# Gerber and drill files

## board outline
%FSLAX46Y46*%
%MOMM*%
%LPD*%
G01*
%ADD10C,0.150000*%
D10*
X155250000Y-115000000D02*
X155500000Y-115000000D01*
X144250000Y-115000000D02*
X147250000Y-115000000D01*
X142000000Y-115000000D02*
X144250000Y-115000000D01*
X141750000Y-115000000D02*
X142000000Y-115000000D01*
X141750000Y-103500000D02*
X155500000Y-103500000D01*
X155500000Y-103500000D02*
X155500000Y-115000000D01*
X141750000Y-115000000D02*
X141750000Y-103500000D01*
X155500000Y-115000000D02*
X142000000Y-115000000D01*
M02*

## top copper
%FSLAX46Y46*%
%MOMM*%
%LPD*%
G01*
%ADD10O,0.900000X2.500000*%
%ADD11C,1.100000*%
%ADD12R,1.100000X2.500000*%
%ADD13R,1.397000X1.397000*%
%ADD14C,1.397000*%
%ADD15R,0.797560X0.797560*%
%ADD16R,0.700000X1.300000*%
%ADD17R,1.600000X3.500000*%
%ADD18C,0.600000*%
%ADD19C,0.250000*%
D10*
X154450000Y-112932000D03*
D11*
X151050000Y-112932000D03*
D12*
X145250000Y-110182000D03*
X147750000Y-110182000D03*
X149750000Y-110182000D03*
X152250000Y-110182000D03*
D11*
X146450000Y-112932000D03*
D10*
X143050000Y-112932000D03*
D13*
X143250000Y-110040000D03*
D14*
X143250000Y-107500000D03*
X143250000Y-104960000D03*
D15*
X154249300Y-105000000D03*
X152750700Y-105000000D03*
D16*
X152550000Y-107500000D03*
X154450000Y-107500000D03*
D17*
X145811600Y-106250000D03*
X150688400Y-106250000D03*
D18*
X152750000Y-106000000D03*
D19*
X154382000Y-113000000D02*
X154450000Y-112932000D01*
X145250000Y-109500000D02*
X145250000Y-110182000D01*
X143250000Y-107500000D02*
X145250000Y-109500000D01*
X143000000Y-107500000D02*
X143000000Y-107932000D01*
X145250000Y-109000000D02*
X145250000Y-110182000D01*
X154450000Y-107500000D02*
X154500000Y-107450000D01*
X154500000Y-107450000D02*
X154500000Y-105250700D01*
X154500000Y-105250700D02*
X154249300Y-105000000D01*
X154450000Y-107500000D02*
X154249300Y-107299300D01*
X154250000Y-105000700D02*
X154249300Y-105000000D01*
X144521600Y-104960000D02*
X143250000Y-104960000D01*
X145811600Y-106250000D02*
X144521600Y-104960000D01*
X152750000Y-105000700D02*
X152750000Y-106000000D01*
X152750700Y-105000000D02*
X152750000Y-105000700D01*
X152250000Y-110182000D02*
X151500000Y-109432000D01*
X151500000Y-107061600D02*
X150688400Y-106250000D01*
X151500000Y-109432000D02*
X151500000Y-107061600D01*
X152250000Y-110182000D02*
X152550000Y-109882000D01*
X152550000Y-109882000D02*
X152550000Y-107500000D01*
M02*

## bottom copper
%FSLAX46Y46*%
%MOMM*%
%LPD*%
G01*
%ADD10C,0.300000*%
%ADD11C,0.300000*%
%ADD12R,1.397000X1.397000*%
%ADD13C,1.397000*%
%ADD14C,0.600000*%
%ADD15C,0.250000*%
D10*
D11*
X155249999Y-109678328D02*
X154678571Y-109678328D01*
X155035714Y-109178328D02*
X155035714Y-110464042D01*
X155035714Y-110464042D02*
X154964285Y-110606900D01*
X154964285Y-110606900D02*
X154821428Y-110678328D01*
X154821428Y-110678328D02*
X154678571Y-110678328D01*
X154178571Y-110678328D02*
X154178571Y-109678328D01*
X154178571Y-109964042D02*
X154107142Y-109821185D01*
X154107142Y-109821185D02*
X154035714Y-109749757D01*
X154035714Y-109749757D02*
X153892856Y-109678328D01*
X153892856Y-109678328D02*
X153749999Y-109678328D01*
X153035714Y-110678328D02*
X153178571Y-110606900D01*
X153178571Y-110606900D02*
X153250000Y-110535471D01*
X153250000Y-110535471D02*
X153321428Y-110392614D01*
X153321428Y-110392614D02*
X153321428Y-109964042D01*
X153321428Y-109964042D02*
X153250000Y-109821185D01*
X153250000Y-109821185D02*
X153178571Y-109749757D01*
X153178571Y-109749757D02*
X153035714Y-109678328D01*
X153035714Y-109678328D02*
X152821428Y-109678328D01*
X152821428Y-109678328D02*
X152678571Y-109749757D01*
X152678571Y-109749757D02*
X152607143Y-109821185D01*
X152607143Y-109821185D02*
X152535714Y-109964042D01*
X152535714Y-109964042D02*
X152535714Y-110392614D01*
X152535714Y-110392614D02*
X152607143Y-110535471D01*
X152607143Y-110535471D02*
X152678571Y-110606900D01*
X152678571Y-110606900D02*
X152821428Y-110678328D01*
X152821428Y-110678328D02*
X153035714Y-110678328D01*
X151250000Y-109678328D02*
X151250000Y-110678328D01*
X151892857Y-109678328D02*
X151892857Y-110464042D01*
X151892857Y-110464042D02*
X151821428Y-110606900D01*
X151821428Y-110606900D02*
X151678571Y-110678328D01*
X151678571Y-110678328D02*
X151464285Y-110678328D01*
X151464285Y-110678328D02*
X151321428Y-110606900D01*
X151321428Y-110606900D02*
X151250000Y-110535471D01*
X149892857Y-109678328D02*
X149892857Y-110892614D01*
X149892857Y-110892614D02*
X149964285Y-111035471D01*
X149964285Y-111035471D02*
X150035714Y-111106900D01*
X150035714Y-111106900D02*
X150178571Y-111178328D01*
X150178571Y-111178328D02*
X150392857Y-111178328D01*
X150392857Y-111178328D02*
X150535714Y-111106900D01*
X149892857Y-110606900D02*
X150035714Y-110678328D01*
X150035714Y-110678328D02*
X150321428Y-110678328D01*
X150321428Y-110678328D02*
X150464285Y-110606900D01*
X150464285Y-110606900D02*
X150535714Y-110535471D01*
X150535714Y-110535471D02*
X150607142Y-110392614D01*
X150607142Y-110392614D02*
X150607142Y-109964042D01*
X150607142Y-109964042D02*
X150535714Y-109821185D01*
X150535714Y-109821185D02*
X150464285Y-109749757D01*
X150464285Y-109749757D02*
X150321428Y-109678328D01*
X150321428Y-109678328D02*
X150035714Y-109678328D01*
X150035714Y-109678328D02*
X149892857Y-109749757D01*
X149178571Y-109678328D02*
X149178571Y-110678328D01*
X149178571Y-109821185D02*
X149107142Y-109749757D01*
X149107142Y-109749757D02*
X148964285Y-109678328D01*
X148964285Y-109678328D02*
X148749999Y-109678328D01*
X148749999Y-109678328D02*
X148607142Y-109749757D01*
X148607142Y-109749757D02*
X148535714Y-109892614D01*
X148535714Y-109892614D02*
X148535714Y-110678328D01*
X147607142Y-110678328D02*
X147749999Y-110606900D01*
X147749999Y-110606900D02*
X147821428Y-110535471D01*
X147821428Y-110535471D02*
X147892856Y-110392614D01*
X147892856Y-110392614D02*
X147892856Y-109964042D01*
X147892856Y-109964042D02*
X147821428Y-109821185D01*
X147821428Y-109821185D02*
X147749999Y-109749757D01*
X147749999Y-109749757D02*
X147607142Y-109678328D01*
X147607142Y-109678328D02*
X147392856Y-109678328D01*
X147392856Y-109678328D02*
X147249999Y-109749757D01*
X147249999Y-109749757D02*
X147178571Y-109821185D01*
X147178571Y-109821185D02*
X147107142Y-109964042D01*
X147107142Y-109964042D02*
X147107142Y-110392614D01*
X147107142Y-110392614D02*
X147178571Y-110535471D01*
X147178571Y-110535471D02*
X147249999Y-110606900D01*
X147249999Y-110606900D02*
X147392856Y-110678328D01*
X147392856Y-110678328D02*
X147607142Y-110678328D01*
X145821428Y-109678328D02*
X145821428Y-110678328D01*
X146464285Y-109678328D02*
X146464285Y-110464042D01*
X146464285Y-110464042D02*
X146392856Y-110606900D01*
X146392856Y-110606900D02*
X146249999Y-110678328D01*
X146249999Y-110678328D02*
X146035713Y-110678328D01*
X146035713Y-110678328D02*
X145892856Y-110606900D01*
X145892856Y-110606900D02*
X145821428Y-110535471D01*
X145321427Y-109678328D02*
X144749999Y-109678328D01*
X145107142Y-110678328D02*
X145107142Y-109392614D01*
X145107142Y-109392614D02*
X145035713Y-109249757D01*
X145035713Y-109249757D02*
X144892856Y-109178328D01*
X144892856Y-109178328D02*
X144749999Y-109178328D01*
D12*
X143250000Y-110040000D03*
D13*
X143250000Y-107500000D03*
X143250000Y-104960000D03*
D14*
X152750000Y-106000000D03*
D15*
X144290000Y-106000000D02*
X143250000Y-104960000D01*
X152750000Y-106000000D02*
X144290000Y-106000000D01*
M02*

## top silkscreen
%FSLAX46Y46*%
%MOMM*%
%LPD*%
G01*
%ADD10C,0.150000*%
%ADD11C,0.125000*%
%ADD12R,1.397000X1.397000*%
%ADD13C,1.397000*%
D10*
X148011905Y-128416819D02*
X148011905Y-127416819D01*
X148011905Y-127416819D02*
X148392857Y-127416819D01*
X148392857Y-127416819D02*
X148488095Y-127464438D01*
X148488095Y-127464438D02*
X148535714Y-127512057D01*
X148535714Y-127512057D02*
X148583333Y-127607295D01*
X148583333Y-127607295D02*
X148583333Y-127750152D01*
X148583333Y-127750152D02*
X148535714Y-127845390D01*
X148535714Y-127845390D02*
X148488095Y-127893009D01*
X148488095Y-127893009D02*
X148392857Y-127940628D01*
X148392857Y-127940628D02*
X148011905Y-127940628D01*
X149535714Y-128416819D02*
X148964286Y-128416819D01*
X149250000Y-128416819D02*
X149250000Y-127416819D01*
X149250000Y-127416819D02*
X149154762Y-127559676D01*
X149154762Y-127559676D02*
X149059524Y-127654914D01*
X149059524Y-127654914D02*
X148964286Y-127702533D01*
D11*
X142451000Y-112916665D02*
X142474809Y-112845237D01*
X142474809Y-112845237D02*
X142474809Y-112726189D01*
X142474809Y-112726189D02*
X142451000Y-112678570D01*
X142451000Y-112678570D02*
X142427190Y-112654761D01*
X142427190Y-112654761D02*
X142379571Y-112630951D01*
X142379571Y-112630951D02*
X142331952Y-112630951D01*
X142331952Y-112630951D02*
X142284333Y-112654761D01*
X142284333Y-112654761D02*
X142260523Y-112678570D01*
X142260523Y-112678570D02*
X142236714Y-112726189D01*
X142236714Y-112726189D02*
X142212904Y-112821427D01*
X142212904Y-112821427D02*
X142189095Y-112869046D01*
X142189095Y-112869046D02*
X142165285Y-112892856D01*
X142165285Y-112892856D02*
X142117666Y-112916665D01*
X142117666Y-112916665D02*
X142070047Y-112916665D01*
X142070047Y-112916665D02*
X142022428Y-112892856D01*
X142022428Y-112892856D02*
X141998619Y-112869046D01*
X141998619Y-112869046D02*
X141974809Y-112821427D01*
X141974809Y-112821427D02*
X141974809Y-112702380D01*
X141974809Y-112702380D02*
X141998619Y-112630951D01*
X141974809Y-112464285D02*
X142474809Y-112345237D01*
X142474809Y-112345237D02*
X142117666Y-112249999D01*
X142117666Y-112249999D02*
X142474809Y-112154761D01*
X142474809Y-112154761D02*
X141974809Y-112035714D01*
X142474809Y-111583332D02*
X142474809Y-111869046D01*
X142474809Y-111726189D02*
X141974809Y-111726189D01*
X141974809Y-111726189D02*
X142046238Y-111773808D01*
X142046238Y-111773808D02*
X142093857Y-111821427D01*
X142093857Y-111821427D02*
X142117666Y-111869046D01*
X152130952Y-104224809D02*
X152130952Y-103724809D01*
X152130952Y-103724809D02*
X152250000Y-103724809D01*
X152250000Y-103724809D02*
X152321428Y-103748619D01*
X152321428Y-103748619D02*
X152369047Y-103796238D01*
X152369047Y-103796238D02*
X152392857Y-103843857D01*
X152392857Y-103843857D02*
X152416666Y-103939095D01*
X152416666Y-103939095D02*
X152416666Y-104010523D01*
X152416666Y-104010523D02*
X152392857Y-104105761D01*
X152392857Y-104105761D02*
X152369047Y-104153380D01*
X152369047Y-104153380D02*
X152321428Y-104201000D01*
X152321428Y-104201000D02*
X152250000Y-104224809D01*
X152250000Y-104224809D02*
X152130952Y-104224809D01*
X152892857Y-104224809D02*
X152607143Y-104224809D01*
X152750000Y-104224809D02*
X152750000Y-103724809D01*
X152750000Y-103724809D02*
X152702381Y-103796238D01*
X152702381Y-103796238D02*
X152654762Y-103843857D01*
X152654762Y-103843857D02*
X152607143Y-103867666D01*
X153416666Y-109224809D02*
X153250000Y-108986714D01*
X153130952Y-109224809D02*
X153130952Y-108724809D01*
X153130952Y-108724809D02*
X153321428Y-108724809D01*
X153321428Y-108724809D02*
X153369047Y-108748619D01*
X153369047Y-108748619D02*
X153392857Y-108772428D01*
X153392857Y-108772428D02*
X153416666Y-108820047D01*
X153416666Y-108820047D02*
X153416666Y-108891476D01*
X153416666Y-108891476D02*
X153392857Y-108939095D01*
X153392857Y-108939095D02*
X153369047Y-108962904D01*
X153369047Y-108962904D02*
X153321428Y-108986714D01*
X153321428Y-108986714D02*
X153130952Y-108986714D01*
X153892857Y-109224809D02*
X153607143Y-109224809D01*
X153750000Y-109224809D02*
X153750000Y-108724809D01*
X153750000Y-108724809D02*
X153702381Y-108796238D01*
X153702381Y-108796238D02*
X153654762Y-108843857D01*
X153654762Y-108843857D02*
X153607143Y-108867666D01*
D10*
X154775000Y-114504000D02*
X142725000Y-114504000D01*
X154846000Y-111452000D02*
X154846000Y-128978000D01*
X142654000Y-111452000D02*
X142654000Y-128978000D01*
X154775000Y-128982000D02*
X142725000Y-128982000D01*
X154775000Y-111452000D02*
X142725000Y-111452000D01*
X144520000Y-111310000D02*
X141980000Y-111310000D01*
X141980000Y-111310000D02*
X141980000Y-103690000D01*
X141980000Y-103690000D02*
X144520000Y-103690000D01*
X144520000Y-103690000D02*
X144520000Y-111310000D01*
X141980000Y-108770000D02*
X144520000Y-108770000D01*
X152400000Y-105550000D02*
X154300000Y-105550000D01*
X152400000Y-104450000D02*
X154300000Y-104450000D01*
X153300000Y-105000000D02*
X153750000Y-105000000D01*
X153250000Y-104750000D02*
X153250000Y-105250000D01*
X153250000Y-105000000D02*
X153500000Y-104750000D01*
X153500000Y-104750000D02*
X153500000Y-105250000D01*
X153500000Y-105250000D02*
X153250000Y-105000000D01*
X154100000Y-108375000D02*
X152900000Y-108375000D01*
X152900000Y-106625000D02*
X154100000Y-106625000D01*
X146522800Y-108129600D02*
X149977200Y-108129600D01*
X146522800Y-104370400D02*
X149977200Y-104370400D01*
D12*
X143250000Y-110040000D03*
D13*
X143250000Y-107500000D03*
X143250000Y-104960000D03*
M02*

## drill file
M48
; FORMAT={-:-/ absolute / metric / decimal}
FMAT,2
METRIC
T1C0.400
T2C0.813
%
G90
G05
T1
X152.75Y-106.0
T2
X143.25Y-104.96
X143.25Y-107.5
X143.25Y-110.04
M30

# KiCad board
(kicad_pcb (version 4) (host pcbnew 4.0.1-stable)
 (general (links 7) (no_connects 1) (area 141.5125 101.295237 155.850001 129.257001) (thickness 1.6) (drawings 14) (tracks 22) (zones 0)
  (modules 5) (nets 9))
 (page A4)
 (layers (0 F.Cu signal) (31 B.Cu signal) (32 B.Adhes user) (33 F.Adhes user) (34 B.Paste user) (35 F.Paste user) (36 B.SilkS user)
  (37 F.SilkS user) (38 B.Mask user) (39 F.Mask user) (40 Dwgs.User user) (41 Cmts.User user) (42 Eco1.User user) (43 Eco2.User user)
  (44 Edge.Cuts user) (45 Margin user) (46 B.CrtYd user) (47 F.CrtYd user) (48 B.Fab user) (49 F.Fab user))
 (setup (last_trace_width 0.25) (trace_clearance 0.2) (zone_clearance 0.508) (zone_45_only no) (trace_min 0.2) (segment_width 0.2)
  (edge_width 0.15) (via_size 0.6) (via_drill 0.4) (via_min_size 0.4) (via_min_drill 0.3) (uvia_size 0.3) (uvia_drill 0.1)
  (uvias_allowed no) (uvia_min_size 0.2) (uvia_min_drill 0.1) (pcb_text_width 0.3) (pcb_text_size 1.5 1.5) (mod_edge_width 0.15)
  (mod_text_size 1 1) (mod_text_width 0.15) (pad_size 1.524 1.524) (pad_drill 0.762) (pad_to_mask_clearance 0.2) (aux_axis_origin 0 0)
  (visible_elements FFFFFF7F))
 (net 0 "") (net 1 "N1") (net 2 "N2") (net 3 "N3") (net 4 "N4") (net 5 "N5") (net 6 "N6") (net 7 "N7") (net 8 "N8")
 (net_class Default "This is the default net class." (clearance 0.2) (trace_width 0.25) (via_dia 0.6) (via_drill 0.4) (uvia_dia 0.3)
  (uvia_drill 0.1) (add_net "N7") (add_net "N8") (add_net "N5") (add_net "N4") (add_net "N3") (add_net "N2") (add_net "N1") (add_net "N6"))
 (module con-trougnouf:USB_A (layer F.Cu) (at 148.75 114.5)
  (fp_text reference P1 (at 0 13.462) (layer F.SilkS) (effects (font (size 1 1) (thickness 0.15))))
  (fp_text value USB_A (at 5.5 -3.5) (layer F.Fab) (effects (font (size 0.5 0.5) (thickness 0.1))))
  (fp_line (start 6.025 0.004) (end -6.025 0.004) (layer F.SilkS) (width 0.15))
  (fp_line (start 6.096 -3.048) (end 6.096 14.478) (layer F.SilkS) (width 0.15))
  (fp_line (start -6.096 -3.048) (end -6.096 14.478) (layer F.SilkS) (width 0.15))
  (fp_line (start 6.025 14.482) (end -6.025 14.482) (layer F.SilkS) (width 0.15))
  (fp_line (start 6.025 -3.048) (end -6.025 -3.048) (layer F.SilkS) (width 0.15))
  (pad 5 smd oval (at 5.7 -1.568) (size 0.9 2.5) (layers F.Cu F.Paste F.Mask) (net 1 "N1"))
  (pad "" smd circle (at 2.3 -1.568) (size 1.1 1.1) (layers F.Cu F.Paste F.Mask))
  (pad 4 smd rect (at -3.5 -4.318) (size 1.1 2.5) (layers F.Cu F.Paste F.Mask) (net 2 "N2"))
  (pad 3 smd rect (at -1 -4.318) (size 1.1 2.5) (layers F.Cu F.Paste F.Mask) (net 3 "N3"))
  (pad 2 smd rect (at 1 -4.318) (size 1.1 2.5) (layers F.Cu F.Paste F.Mask) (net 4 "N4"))
  (pad 1 smd rect (at 3.5 -4.318) (size 1.1 2.5) (layers F.Cu F.Paste F.Mask) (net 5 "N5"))
  (pad "" smd circle (at -2.3 -1.568) (size 1.1 1.1) (layers F.Cu F.Paste F.Mask))
  (pad 5 smd oval (at -5.7 -1.568) (size 0.9 2.5) (layers F.Cu F.Paste F.Mask) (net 1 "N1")))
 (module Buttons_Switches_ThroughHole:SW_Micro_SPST (layer F.Cu) (at 143.25 107.5 90)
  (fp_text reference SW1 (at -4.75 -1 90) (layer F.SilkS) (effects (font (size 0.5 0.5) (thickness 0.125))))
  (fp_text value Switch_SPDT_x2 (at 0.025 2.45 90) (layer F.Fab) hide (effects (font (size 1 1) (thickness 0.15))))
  (fp_line (start -3.81 1.27) (end -3.81 -1.27) (layer F.SilkS) (width 0.15))
  (fp_line (start -3.81 -1.27) (end 3.81 -1.27) (layer F.SilkS) (width 0.15))
  (fp_line (start 3.81 -1.27) (end 3.81 1.27) (layer F.SilkS) (width 0.15))
  (fp_line (start 3.81 1.27) (end -3.81 1.27) (layer F.SilkS) (width 0.15))
  (fp_line (start -1.27 -1.27) (end -1.27 1.27) (layer F.SilkS) (width 0.15))
  (pad 1 thru_hole rect (at -2.54 0 90) (size 1.397 1.397) (drill 0.8128) (layers *.Cu *.Mask F.SilkS) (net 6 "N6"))
  (pad 2 thru_hole circle (at 0 0 90) (size 1.397 1.397) (drill 0.8128) (layers *.Cu *.Mask F.SilkS) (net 2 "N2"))
  (pad 3 thru_hole circle (at 2.54 0 90) (size 1.397 1.397) (drill 0.8128) (layers *.Cu *.Mask F.SilkS) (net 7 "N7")))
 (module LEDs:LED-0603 (layer F.Cu) (at 153.5 105)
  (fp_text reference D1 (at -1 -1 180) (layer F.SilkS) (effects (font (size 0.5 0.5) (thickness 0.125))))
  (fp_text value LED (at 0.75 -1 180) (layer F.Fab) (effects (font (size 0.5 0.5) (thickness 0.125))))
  (fp_line (start -1.1 0.55) (end 0.8 0.55) (layer F.SilkS) (width 0.15))
  (fp_line (start -1.1 -0.55) (end 0.8 -0.55) (layer F.SilkS) (width 0.15))
  (fp_line (start -0.2 0) (end 0.25 0) (layer F.SilkS) (width 0.15))
  (fp_line (start -0.25 -0.25) (end -0.25 0.25) (layer F.SilkS) (width 0.15))
  (fp_line (start -0.25 0) (end 0 -0.25) (layer F.SilkS) (width 0.15))
  (fp_line (start 0 -0.25) (end 0 0.25) (layer F.SilkS) (width 0.15))
  (fp_line (start 0 0.25) (end -0.25 0) (layer F.SilkS) (width 0.15))
  (pad 2 smd rect (at 0.7493 0 180) (size 0.79756 0.79756) (layers F.Cu F.Paste F.Mask) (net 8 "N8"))
  (pad 1 smd rect (at -0.7493 0 180) (size 0.79756 0.79756) (layers F.Cu F.Paste F.Mask) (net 7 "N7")))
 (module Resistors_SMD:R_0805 (layer F.Cu) (at 153.5 107.5)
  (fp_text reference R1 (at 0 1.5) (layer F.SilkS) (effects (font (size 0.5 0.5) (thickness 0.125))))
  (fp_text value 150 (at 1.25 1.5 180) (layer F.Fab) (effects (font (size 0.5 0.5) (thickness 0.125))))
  (fp_line (start 0.6 0.875) (end -0.6 0.875) (layer F.SilkS) (width 0.15))
  (fp_line (start -0.6 -0.875) (end 0.6 -0.875) (layer F.SilkS) (width 0.15))
  (pad 1 smd rect (at -0.95 0) (size 0.7 1.3) (layers F.Cu F.Paste F.Mask) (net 5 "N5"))
  (pad 2 smd rect (at 0.95 0) (size 0.7 1.3) (layers F.Cu F.Paste F.Mask) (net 8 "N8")))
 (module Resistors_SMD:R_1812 (layer F.Cu) (at 148.25 106.25)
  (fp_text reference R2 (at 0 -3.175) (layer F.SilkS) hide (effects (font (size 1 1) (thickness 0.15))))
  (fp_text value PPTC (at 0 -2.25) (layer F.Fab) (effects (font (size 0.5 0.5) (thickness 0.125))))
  (fp_line (start -1.7272 1.8796) (end 1.7272 1.8796) (layer F.SilkS) (width 0.15))
  (fp_line (start -1.7272 -1.8796) (end 1.7272 -1.8796) (layer F.SilkS) (width 0.15))
  (pad 1 smd rect (at -2.4384 0) (size 1.6 3.5) (layers F.Cu F.Paste F.Mask) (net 7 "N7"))
  (pad 2 smd rect (at 2.4384 0) (size 1.6 3.5) (layers F.Cu F.Paste F.Mask) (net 5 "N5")))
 (gr_line (start 155.25 115) (end 155.5 115) (angle 90) (layer Edge.Cuts) (width 0.15))
 (gr_line (start 144.25 115) (end 147.25 115) (angle 90) (layer Edge.Cuts) (width 0.15))
 (gr_line (start 142 115) (end 144.25 115) (angle 90) (layer Edge.Cuts) (width 0.15))
 (gr_line (start 141.75 115) (end 142 115) (angle 90) (layer Edge.Cuts) (width 0.15))
 (gr_line (start 141.75 103.5) (end 155.5 103.5) (angle 90) (layer Edge.Cuts) (width 0.15))
 (gr_line (start 155.5 103.5) (end 155.5 115) (angle 90) (layer Edge.Cuts) (width 0.15))
 (gr_line (start 141.75 115) (end 141.75 103.5) (angle 90) (layer Edge.Cuts) (width 0.15))
 (gr_line (start 155.5 115) (end 142 115) (angle 90) (layer Edge.Cuts) (width 0.15))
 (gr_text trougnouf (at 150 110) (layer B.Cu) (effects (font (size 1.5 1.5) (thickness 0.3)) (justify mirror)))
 (segment (start 154.382 113) (end 154.45 112.932) (width 0.25) (layer F.Cu) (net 1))
 (segment (start 145.25 109.5) (end 145.25 110.182) (width 0.25) (layer F.Cu) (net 2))
 (segment (start 143.25 107.5) (end 145.25 109.5) (width 0.25) (layer F.Cu) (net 2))
 (segment (start 143 107.5) (end 143 107.932) (width 0.25) (layer F.Cu) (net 2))
 (segment (start 145.25 109) (end 145.25 110.182) (width 0.25) (layer F.Cu) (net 2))
 (segment (start 154.45 107.5) (end 154.5 107.45) (width 0.25) (layer F.Cu) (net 8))
 (segment (start 154.5 107.45) (end 154.5 105.2507) (width 0.25) (layer F.Cu) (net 8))
 (segment (start 154.5 105.2507) (end 154.2493 105) (width 0.25) (layer F.Cu) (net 8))
 (segment (start 154.45 107.5) (end 154.2493 107.2993) (width 0.25) (layer F.Cu) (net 8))
 (segment (start 154.25 105.0007) (end 154.2493 105) (width 0.25) (layer F.Cu) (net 8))
 (segment (start 144.5216 104.96) (end 143.25 104.96) (width 0.25) (layer F.Cu) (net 7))
 (segment (start 145.8116 106.25) (end 144.5216 104.96) (width 0.25) (layer F.Cu) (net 7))
 (segment (start 144.29 106) (end 143.25 104.96) (width 0.25) (layer B.Cu) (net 7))
 (segment (start 152.75 106) (end 144.29 106) (width 0.25) (layer B.Cu) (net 7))
 (via (at 152.75 106) (size 0.6) (drill 0.4) (layers F.Cu B.Cu) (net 7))
 (segment (start 152.75 105.0007) (end 152.75 106) (width 0.25) (layer F.Cu) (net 7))
 (segment (start 152.7507 105) (end 152.75 105.0007) (width 0.25) (layer F.Cu) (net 7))
 (segment (start 152.25 110.182) (end 151.5 109.432) (width 0.25) (layer F.Cu) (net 5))
 (segment (start 151.5 107.0616) (end 150.6884 106.25) (width 0.25) (layer F.Cu) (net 5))
 (segment (start 151.5 109.432) (end 151.5 107.0616) (width 0.25) (layer F.Cu) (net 5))
 (segment (start 152.25 110.182) (end 152.55 109.882) (width 0.25) (layer F.Cu) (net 5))
 (segment (start 152.55 109.882) (end 152.55 107.5) (width 0.25) (layer F.Cu) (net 5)))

